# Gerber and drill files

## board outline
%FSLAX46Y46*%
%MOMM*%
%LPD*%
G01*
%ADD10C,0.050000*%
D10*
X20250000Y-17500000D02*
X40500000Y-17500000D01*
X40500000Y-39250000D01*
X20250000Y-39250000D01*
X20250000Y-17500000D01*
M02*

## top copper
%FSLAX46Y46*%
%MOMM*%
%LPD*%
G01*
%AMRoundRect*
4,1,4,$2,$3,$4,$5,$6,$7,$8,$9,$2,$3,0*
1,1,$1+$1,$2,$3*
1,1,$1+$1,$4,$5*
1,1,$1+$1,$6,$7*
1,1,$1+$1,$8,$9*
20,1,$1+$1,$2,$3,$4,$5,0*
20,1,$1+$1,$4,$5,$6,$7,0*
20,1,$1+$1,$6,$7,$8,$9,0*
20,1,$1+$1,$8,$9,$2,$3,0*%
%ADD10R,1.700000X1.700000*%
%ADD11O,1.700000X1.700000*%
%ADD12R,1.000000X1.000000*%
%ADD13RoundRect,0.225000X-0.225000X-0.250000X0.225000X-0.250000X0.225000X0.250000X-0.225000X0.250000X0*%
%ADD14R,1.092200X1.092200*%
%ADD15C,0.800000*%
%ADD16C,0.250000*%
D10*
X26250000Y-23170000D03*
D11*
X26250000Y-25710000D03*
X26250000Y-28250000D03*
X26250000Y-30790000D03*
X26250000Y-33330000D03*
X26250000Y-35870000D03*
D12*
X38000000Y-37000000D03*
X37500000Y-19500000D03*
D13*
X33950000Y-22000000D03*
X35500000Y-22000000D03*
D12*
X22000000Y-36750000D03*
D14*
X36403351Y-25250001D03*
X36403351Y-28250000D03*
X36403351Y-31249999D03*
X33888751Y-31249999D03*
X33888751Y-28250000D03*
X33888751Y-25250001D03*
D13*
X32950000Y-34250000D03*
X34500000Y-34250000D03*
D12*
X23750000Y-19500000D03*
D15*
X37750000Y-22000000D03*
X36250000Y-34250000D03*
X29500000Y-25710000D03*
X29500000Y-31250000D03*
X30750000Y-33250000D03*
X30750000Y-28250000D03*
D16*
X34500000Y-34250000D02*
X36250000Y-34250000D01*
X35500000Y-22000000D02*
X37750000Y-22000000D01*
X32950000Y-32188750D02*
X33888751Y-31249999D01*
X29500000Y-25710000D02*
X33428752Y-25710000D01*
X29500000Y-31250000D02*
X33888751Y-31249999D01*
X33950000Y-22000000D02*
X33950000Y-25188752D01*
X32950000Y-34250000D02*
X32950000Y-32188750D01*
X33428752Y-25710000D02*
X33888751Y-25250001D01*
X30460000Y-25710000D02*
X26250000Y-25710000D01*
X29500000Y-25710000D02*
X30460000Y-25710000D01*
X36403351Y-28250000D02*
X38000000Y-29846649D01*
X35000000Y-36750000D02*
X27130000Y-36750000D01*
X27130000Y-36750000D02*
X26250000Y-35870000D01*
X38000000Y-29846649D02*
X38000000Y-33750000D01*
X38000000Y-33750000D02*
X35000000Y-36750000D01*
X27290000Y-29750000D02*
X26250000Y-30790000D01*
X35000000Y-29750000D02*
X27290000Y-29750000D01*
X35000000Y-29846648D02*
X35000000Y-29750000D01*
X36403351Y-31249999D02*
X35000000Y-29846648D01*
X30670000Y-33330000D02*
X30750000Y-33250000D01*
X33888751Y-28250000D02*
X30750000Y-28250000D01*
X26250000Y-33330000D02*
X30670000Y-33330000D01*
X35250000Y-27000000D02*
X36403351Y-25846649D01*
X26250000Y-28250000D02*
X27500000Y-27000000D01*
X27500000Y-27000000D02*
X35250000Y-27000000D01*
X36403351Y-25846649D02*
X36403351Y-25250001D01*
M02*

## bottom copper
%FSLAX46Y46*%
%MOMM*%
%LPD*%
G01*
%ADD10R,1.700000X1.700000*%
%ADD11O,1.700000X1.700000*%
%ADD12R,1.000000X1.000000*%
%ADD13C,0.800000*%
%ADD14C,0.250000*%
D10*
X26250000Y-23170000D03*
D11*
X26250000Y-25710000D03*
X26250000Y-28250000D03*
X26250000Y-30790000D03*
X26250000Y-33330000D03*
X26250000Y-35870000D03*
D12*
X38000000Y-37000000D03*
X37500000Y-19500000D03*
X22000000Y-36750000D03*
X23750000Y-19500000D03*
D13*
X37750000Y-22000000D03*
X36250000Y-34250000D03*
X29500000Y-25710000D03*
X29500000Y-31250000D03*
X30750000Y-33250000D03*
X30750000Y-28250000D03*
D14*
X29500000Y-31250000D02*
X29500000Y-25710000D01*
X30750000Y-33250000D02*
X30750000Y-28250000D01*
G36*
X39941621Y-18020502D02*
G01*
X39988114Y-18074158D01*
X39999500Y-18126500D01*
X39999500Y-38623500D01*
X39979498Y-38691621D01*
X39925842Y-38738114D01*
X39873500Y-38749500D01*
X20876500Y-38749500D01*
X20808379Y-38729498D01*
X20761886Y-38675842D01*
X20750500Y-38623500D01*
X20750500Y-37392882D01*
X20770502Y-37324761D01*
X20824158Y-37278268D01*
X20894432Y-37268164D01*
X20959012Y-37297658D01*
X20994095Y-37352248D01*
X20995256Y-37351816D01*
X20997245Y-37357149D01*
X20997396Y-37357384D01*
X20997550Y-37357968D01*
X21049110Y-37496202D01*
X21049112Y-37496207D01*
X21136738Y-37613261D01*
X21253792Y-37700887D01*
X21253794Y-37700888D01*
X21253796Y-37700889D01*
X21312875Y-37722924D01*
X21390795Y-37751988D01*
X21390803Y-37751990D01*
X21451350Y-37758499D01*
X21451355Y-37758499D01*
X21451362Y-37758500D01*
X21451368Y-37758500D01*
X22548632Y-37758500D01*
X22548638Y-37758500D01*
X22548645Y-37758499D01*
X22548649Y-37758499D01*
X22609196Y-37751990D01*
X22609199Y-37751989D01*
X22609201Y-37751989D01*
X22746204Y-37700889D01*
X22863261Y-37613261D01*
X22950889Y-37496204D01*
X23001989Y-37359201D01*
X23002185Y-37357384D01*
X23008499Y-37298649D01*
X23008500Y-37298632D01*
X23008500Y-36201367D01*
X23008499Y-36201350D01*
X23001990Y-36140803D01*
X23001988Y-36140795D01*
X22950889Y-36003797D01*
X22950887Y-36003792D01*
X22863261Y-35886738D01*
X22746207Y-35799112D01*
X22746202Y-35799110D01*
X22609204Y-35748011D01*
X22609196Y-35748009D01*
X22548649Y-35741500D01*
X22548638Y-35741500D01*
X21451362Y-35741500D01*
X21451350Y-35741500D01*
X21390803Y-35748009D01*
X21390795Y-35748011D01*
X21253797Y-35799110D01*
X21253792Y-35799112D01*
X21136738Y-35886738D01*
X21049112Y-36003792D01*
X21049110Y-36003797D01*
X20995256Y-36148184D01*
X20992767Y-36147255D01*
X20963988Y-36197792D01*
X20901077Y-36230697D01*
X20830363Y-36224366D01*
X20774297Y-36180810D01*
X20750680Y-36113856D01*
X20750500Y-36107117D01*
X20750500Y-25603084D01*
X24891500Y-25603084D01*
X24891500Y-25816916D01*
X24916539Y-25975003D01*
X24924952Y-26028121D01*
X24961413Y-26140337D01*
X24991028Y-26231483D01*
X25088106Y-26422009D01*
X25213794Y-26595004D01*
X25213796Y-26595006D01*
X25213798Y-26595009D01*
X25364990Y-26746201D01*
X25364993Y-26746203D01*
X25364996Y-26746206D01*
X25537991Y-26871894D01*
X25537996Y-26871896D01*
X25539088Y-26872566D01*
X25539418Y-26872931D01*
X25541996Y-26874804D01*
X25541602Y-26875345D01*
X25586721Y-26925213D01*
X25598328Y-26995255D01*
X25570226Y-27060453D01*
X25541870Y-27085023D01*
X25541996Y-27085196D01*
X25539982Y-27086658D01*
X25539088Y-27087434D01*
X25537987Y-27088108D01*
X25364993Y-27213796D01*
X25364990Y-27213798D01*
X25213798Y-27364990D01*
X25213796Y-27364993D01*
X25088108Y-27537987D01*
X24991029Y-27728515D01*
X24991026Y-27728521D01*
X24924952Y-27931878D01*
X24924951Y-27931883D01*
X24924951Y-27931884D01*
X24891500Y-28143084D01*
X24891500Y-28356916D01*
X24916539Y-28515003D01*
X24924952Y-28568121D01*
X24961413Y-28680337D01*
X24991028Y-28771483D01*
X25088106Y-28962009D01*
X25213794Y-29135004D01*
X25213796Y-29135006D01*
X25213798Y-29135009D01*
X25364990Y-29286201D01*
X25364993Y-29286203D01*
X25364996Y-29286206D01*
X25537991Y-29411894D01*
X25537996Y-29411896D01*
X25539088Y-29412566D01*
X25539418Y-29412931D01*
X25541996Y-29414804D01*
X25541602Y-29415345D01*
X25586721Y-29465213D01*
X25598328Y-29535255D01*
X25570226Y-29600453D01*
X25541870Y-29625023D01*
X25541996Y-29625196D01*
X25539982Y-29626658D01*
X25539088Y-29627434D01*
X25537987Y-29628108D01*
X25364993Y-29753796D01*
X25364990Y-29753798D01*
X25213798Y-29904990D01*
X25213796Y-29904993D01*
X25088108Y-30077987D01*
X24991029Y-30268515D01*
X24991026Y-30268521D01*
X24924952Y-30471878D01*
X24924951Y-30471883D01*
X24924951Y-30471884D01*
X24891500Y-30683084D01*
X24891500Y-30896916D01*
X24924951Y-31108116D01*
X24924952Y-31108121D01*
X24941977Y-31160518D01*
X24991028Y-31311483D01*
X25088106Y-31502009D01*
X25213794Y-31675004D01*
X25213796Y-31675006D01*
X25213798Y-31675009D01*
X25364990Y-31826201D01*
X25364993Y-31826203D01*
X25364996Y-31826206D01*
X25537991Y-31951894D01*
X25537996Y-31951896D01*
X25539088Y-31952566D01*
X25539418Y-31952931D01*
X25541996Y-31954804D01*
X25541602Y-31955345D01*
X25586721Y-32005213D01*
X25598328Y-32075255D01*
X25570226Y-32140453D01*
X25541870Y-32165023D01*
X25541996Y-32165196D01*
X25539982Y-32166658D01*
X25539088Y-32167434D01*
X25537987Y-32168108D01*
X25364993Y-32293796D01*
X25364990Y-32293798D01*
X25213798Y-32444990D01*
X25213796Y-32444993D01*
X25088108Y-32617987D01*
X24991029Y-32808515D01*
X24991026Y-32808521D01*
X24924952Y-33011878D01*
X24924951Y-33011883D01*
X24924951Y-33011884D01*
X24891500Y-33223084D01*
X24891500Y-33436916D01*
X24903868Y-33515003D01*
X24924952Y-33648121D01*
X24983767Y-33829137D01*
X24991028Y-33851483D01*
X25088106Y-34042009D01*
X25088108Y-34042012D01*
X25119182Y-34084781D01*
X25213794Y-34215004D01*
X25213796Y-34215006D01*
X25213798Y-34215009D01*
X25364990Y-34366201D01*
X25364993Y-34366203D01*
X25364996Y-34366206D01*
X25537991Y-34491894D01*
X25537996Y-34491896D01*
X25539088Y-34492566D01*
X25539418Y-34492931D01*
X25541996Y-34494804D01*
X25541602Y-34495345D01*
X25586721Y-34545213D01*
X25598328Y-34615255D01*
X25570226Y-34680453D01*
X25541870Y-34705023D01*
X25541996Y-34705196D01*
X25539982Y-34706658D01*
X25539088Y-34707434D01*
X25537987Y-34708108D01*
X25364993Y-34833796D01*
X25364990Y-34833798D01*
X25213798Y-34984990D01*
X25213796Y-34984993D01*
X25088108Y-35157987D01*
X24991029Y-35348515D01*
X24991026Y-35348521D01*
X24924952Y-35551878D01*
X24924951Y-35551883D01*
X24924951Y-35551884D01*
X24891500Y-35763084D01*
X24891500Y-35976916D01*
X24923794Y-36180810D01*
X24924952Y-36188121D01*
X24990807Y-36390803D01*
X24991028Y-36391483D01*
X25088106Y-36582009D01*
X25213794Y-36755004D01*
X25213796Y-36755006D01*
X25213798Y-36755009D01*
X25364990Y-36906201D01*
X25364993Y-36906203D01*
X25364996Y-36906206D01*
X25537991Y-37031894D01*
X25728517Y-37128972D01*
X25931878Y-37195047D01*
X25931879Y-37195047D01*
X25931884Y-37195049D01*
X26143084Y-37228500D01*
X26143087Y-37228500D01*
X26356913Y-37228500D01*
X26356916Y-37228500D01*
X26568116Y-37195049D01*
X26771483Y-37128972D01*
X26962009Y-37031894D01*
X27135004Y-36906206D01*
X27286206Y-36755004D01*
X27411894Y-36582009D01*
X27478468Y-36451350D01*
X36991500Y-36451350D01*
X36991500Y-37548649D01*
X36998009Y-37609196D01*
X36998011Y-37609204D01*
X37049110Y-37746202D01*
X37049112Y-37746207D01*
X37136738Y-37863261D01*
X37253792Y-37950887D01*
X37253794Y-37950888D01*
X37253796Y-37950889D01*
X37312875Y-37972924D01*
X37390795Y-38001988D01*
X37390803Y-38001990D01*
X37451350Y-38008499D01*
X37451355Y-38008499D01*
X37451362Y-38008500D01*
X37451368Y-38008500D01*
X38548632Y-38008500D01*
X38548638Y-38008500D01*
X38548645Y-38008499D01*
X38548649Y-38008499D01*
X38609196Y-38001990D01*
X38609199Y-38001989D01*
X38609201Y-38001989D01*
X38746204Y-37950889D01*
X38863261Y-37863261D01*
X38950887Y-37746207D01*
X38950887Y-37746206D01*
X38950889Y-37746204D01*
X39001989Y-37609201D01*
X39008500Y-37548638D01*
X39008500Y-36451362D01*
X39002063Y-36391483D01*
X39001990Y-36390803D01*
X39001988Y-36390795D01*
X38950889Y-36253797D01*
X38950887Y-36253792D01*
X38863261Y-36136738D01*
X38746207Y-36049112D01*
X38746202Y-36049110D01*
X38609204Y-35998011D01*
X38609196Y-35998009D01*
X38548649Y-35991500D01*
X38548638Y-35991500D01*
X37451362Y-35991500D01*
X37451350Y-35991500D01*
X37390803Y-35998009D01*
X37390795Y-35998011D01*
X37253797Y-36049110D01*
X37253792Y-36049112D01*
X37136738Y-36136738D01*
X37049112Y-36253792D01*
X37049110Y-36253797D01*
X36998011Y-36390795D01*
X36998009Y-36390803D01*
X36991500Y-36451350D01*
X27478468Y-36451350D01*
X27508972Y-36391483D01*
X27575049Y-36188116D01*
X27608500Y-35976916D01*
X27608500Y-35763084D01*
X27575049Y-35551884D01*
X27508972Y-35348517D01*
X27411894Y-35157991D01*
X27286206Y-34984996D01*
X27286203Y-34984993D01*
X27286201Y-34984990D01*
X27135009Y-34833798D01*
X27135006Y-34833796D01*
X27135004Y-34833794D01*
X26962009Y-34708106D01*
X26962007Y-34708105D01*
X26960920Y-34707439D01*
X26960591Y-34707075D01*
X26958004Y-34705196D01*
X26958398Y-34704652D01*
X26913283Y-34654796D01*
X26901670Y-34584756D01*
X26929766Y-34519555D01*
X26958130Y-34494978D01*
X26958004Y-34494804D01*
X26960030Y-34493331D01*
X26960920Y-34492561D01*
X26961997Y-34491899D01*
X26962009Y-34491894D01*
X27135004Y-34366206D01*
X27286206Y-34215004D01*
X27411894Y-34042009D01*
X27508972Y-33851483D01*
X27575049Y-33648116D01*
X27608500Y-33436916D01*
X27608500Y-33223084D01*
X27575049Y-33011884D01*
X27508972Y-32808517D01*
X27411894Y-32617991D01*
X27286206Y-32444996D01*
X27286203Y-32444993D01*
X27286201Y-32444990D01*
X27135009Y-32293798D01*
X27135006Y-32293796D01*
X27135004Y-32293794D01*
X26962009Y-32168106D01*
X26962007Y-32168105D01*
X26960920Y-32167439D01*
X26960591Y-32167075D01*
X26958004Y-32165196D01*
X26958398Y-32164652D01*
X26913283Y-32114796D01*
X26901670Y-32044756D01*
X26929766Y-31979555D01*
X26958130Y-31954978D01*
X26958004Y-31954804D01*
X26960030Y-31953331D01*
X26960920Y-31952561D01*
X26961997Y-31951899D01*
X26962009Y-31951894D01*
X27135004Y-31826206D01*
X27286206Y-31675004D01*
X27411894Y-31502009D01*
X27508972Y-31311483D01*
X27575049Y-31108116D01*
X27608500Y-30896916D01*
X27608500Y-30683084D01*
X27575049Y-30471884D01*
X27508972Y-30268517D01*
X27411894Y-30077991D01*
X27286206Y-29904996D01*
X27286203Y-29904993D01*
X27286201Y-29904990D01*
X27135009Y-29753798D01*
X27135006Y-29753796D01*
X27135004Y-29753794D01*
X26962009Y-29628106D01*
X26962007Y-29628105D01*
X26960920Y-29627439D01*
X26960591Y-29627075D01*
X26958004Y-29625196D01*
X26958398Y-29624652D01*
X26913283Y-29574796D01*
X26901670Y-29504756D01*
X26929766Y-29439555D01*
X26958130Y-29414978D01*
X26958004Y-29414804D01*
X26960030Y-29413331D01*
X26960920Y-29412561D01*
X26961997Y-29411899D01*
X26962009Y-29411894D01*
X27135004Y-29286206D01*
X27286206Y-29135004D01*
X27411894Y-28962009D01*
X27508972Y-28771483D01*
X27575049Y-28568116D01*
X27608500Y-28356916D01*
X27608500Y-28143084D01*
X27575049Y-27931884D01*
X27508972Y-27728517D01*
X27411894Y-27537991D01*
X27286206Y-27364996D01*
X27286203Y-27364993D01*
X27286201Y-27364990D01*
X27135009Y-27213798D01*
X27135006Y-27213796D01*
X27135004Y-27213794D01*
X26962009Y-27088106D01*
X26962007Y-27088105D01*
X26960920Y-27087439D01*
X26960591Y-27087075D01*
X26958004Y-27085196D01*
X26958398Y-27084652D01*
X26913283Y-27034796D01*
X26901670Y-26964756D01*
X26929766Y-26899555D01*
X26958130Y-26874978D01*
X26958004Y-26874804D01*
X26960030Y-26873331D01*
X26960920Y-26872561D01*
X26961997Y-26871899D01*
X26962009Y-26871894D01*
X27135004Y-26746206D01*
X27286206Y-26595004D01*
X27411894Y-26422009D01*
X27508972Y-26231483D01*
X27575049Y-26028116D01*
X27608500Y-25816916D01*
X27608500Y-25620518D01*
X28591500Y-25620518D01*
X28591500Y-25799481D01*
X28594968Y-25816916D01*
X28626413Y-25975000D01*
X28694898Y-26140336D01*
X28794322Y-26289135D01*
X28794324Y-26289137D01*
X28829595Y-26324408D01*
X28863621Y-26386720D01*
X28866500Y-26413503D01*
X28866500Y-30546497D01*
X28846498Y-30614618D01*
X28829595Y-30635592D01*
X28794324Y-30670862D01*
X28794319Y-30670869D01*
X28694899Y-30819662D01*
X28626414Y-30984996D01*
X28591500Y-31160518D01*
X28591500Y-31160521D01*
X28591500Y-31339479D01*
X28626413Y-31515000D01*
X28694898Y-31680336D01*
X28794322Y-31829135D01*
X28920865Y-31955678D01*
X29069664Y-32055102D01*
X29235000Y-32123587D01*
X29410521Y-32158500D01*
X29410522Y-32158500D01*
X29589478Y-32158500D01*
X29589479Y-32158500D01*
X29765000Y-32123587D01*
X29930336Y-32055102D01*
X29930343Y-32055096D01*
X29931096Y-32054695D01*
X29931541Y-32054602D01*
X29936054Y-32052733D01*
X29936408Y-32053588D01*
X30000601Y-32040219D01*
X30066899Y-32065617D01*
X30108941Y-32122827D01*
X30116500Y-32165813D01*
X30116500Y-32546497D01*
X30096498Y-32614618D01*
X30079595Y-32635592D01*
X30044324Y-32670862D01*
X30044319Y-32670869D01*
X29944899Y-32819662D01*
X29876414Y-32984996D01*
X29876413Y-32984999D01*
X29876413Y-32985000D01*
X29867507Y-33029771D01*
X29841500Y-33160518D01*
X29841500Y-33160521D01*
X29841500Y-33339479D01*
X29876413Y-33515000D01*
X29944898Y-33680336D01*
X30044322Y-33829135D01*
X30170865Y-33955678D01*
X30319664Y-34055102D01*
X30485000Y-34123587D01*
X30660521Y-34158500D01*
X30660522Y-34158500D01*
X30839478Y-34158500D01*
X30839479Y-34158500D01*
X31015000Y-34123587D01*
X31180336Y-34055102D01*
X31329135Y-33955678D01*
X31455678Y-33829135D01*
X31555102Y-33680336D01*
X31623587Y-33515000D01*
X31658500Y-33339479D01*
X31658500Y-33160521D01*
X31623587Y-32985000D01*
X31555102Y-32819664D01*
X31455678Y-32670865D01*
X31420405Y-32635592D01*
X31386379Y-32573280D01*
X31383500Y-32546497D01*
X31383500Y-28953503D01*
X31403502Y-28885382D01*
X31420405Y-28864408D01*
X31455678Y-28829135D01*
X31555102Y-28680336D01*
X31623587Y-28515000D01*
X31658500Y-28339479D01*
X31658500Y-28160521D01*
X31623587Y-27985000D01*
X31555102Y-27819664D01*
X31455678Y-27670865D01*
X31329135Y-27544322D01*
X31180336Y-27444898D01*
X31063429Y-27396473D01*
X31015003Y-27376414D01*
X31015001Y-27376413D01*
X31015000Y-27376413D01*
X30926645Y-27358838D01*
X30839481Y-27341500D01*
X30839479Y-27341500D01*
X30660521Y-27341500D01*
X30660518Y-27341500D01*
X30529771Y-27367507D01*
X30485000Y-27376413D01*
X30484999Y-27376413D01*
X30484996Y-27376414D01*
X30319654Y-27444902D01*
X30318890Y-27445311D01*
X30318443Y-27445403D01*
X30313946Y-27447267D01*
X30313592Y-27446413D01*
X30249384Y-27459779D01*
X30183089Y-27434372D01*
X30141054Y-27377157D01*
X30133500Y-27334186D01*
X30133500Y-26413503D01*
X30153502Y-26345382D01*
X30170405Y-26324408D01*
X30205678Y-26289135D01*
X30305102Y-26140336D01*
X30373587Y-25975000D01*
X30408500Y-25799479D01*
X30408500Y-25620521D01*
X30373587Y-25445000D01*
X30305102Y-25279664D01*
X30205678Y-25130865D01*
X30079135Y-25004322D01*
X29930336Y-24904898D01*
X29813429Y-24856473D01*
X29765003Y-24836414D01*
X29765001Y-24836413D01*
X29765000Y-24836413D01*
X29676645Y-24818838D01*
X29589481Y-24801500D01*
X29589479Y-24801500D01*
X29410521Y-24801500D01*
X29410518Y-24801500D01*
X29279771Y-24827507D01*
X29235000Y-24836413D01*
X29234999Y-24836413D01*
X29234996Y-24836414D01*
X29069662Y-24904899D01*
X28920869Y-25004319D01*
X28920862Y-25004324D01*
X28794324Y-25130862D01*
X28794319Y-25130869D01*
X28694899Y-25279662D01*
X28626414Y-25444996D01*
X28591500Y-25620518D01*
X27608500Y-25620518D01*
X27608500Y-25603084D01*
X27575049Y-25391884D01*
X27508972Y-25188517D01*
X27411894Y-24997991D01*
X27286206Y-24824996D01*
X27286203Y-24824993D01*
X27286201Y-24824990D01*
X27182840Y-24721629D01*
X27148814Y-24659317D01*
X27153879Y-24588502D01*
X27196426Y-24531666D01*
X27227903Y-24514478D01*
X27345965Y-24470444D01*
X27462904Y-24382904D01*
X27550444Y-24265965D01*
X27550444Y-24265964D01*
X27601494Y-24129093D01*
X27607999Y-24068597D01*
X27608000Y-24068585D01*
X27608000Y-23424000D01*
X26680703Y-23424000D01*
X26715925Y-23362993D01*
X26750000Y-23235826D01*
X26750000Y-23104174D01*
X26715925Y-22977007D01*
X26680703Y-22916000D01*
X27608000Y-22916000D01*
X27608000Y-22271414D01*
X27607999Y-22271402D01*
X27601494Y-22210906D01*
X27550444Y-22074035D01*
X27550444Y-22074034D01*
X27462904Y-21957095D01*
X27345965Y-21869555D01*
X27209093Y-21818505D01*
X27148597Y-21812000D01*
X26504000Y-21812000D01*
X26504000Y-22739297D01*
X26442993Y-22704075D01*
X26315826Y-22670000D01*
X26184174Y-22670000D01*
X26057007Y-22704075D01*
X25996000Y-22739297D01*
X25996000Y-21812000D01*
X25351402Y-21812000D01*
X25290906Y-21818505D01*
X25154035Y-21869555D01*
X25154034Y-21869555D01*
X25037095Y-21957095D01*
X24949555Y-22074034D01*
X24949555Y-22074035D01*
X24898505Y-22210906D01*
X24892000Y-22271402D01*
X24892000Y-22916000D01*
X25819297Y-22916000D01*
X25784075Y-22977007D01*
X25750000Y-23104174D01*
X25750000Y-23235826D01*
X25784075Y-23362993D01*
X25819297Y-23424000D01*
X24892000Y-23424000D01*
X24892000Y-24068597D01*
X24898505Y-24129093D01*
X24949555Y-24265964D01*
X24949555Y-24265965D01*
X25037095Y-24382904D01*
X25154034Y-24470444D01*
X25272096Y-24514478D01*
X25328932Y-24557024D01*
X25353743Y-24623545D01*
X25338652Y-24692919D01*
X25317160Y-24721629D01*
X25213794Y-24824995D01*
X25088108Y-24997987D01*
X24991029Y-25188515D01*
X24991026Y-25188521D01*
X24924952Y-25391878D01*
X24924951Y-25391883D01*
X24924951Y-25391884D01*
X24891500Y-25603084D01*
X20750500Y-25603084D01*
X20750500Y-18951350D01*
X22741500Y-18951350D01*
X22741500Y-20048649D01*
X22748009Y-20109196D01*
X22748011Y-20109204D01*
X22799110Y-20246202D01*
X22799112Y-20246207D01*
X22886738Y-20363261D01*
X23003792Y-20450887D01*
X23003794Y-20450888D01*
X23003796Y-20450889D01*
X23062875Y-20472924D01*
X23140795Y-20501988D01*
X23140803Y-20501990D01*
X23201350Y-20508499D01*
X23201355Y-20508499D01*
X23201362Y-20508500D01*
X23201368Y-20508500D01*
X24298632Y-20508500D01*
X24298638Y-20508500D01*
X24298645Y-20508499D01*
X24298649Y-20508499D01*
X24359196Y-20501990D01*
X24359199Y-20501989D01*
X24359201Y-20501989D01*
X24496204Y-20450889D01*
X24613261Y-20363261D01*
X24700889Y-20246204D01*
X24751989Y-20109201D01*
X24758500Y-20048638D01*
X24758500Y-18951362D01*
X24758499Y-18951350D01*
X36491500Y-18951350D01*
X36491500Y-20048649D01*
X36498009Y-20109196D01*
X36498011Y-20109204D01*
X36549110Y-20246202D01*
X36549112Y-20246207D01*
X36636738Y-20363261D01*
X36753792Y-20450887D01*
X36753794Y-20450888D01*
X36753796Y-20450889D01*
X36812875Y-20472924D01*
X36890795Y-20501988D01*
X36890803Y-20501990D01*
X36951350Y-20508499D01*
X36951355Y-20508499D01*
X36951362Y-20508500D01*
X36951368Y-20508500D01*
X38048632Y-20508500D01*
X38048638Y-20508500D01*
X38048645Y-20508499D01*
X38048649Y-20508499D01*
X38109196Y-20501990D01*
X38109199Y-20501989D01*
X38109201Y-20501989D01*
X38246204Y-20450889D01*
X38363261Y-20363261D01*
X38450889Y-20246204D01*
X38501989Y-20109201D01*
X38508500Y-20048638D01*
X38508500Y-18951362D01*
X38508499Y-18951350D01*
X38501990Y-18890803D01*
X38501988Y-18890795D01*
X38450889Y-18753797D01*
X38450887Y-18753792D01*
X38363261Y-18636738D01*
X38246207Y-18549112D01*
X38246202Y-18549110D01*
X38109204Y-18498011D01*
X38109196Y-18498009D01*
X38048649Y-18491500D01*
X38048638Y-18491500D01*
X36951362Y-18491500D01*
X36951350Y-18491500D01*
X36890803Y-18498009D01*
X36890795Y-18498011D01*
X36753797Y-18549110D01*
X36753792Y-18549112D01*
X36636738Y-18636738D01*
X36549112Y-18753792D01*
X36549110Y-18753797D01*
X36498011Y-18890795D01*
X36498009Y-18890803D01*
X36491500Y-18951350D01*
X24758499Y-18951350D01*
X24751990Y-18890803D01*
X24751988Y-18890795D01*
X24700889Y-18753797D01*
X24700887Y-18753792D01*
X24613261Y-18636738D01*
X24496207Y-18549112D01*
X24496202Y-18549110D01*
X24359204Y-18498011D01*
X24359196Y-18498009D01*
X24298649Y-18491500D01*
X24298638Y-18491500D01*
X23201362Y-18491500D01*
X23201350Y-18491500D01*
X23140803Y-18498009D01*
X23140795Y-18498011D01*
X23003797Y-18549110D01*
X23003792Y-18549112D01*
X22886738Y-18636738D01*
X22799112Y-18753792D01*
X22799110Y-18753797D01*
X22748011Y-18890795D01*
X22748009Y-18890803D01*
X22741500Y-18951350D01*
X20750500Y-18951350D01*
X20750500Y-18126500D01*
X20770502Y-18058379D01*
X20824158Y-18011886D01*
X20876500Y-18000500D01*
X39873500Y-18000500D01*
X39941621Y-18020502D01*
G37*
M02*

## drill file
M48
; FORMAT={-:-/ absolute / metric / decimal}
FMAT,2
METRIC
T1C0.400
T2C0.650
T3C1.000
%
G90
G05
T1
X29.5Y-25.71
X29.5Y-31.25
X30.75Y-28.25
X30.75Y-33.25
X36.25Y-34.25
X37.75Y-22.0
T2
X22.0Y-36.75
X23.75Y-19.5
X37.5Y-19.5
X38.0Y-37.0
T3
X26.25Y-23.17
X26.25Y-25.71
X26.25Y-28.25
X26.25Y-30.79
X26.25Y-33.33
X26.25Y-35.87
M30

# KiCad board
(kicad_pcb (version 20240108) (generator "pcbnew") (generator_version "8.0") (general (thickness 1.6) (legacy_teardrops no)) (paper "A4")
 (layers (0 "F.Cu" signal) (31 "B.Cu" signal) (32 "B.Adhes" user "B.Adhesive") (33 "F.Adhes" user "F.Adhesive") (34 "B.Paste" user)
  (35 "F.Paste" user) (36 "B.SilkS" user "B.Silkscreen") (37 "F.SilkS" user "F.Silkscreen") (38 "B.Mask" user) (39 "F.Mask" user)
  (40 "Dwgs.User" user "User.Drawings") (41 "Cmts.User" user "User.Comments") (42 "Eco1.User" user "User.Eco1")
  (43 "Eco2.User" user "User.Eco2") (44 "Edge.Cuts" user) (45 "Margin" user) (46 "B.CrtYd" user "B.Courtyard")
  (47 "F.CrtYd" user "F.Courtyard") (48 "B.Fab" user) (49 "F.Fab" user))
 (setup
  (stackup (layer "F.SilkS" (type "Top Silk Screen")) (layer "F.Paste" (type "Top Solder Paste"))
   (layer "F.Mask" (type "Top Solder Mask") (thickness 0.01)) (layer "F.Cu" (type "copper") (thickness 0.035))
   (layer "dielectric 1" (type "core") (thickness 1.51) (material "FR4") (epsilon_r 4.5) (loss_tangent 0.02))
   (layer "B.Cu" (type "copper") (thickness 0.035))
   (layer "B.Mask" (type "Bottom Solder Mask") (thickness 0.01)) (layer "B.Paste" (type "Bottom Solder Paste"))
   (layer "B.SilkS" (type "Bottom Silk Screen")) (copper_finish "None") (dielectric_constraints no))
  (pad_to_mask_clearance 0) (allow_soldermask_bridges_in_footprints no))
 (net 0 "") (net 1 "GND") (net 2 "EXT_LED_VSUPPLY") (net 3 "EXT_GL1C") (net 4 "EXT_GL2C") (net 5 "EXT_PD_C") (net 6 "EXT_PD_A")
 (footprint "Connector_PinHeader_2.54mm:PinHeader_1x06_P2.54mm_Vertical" (layer "F.Cu") (at 26.25 23.17)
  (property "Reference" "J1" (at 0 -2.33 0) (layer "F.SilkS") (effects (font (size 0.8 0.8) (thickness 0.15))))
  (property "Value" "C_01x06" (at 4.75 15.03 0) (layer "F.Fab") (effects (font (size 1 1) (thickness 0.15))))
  (pad "1" thru_hole rect (at 0 0) (size 1.7 1.7) (drill 1) (layers "*.Cu" "*.Mask") (remove_unused_layers no) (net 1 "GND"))
  (pad "2" thru_hole oval (at 0 2.54) (size 1.7 1.7) (drill 1) (layers "*.Cu" "*.Mask") (remove_unused_layers no) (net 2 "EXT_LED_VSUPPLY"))
  (pad "3" thru_hole oval (at 0 5.08) (size 1.7 1.7) (drill 1) (layers "*.Cu" "*.Mask") (remove_unused_layers no) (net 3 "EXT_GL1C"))
  (pad "4" thru_hole oval (at 0 7.62) (size 1.7 1.7) (drill 1) (layers "*.Cu" "*.Mask") (remove_unused_layers no) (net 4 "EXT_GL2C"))
  (pad "5" thru_hole oval (at 0 10.16) (size 1.7 1.7) (drill 1) (layers "*.Cu" "*.Mask") (remove_unused_layers no) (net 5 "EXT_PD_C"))
  (pad "6" thru_hole oval (at 0 12.7) (size 1.7 1.7) (drill 1) (layers "*.Cu" "*.Mask") (remove_unused_layers no) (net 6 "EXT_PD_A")))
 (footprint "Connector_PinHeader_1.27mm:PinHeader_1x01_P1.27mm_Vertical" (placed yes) (layer "F.Cu") (at 38 37)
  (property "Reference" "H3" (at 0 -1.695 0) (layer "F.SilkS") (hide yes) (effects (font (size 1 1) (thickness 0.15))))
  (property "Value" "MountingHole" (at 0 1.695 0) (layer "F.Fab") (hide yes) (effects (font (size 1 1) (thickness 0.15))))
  (pad "1" thru_hole rect (at 0 0) (size 1 1) (drill 0.65) (layers "*.Cu" "*.Mask") (remove_unused_layers no)))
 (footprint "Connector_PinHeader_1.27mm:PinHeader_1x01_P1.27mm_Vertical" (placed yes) (layer "F.Cu") (at 37.5 19.5 180)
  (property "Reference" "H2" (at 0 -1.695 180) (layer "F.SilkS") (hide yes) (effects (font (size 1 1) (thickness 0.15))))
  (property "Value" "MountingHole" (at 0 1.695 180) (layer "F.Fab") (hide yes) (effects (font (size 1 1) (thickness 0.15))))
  (pad "1" thru_hole rect (at 0 0 180) (size 1 1) (drill 0.65) (layers "*.Cu" "*.Mask") (remove_unused_layers no)))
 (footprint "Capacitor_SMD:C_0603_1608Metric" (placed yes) (layer "F.Cu") (at 34.725 22)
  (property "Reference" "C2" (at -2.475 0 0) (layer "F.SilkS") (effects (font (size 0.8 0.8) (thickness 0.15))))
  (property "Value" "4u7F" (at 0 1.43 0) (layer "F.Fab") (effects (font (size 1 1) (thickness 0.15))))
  (pad "1" smd roundrect (at -0.775 0) (size 0.9 0.95) (layers "F.Cu" "F.Paste" "F.Mask") (roundrect_rratio 0.25) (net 2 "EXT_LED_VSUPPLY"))
  (pad "2" smd roundrect (at 0.775 0) (size 0.9 0.95) (layers "F.Cu" "F.Paste" "F.Mask") (roundrect_rratio 0.25) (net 1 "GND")))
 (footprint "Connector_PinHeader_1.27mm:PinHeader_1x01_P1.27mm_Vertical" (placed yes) (layer "F.Cu") (at 22 36.75 -90)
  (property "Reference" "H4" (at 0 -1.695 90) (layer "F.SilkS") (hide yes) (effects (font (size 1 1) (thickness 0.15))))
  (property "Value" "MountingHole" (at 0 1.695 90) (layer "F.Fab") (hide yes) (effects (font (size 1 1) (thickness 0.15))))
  (pad "1" thru_hole rect (at 0 0 270) (size 1 1) (drill 0.65) (layers "*.Cu" "*.Mask") (remove_unused_layers no)))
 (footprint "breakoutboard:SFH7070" (layer "F.Cu") (at 35.146051 28.25)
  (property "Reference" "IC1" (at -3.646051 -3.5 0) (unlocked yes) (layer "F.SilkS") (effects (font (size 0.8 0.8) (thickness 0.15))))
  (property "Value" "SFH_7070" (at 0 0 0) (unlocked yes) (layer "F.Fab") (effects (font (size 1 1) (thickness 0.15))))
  (pad "1" smd rect (at 1.2573 -2.999999) (size 1.0922 1.0922) (layers "F.Cu" "F.Paste" "F.Mask") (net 3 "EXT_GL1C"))
  (pad "2" smd rect (at 1.2573 0) (size 1.0922 1.0922) (layers "F.Cu" "F.Paste" "F.Mask") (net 6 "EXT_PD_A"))
  (pad "3" smd rect (at 1.2573 2.999999) (size 1.0922 1.0922) (layers "F.Cu" "F.Paste" "F.Mask") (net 4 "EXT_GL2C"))
  (pad "4" smd rect (at -1.2573 2.999999) (size 1.0922 1.0922) (layers "F.Cu" "F.Paste" "F.Mask") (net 2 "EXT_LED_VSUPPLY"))
  (pad "5" smd rect (at -1.2573 0) (size 1.0922 1.0922) (layers "F.Cu" "F.Paste" "F.Mask") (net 5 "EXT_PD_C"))
  (pad "6" smd rect (at -1.2573 -2.999999) (size 1.0922 1.0922) (layers "F.Cu" "F.Paste" "F.Mask") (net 2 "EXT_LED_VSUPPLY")))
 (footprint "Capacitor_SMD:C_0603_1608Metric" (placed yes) (layer "F.Cu") (at 33.725 34.25)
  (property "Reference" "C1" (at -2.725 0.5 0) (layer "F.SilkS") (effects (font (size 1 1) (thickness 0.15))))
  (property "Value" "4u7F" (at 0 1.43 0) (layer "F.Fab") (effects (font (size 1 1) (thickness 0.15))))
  (pad "1" smd roundrect (at -0.775 0) (size 0.9 0.95) (layers "F.Cu" "F.Paste" "F.Mask") (roundrect_rratio 0.25) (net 2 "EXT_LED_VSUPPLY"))
  (pad "2" smd roundrect (at 0.775 0) (size 0.9 0.95) (layers "F.Cu" "F.Paste" "F.Mask") (roundrect_rratio 0.25) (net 1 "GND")))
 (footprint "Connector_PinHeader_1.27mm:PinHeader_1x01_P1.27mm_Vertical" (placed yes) (layer "F.Cu") (at 23.75 19.5)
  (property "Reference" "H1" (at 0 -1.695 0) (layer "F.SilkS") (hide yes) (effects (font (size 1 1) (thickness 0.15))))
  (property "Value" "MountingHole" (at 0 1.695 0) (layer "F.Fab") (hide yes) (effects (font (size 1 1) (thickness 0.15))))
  (pad "1" thru_hole rect (at 0 0) (size 1 1) (drill 0.65) (layers "*.Cu" "*.Mask") (remove_unused_layers no)))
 (gr_rect (start 20.25 17.5) (end 40.5 39.25) (stroke (width 0.05) (type solid)) (fill none) (layer "Edge.Cuts"))
 (segment (start 34.5 34.25) (end 36.25 34.25) (width 0.25) (layer "F.Cu") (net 1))
 (segment (start 35.5 22) (end 37.75 22) (width 0.25) (layer "F.Cu") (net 1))
 (via (at 37.75 22) (size 0.8) (drill 0.4) (layers "F.Cu" "B.Cu") (free yes) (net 1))
 (via (at 36.25 34.25) (size 0.8) (drill 0.4) (layers "F.Cu" "B.Cu") (free yes) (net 1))
 (segment (start 32.95 32.18875) (end 33.888751 31.249999) (width 0.25) (layer "F.Cu") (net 2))
 (segment (start 29.5 25.71) (end 33.428752 25.71) (width 0.25) (layer "F.Cu") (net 2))
 (segment (start 29.5 31.25) (end 33.888751 31.249999) (width 0.25) (layer "F.Cu") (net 2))
 (segment (start 33.95 22) (end 33.95 25.188752) (width 0.25) (layer "F.Cu") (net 2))
 (segment (start 32.95 34.25) (end 32.95 32.18875) (width 0.25) (layer "F.Cu") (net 2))
 (segment (start 33.428752 25.71) (end 33.888751 25.250001) (width 0.25) (layer "F.Cu") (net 2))
 (segment (start 30.46 25.71) (end 26.25 25.71) (width 0.25) (layer "F.Cu") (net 2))
 (segment (start 29.5 25.71) (end 30.46 25.71) (width 0.25) (layer "F.Cu") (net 2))
 (via (at 29.5 25.71) (size 0.8) (drill 0.4) (layers "F.Cu" "B.Cu") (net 2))
 (via (at 29.5 31.25) (size 0.8) (drill 0.4) (layers "F.Cu" "B.Cu") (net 2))
 (segment (start 29.5 31.25) (end 29.5 25.71) (width 0.25) (layer "B.Cu") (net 2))
 (segment (start 36.403351 28.25) (end 38 29.846649) (width 0.25) (layer "F.Cu") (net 6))
 (segment (start 35 36.75) (end 27.13 36.75) (width 0.25) (layer "F.Cu") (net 6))
 (segment (start 27.13 36.75) (end 26.25 35.87) (width 0.25) (layer "F.Cu") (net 6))
 (segment (start 38 29.846649) (end 38 33.75) (width 0.25) (layer "F.Cu") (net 6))
 (segment (start 38 33.75) (end 35 36.75) (width 0.25) (layer "F.Cu") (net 6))
 (segment (start 27.29 29.75) (end 26.25 30.79) (width 0.25) (layer "F.Cu") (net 4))
 (segment (start 35 29.75) (end 27.29 29.75) (width 0.25) (layer "F.Cu") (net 4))
 (segment (start 35 29.846648) (end 35 29.75) (width 0.25) (layer "F.Cu") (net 4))
 (segment (start 36.403351 31.249999) (end 35 29.846648) (width 0.25) (layer "F.Cu") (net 4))
 (segment (start 30.67 33.33) (end 30.75 33.25) (width 0.25) (layer "F.Cu") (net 5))
 (segment (start 33.888751 28.25) (end 30.75 28.25) (width 0.25) (layer "F.Cu") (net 5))
 (segment (start 26.25 33.33) (end 30.67 33.33) (width 0.25) (layer "F.Cu") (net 5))
 (via (at 30.75 33.25) (size 0.8) (drill 0.4) (layers "F.Cu" "B.Cu") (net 5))
 (via (at 30.75 28.25) (size 0.8) (drill 0.4) (layers "F.Cu" "B.Cu") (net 5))
 (segment (start 30.75 33.25) (end 30.75 28.25) (width 0.25) (layer "B.Cu") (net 5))
 (segment (start 35.25 27) (end 36.403351 25.846649) (width 0.25) (layer "F.Cu") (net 3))
 (segment (start 26.25 28.25) (end 27.5 27) (width 0.25) (layer "F.Cu") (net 3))
 (segment (start 27.5 27) (end 35.25 27) (width 0.25) (layer "F.Cu") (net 3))
 (segment (start 36.403351 25.846649) (end 36.403351 25.250001) (width 0.25) (layer "F.Cu") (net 3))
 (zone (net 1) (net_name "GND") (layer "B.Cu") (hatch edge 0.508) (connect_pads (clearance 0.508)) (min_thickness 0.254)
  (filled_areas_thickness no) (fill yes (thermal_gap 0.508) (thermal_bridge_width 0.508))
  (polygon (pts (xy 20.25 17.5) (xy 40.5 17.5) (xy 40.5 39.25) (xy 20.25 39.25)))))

